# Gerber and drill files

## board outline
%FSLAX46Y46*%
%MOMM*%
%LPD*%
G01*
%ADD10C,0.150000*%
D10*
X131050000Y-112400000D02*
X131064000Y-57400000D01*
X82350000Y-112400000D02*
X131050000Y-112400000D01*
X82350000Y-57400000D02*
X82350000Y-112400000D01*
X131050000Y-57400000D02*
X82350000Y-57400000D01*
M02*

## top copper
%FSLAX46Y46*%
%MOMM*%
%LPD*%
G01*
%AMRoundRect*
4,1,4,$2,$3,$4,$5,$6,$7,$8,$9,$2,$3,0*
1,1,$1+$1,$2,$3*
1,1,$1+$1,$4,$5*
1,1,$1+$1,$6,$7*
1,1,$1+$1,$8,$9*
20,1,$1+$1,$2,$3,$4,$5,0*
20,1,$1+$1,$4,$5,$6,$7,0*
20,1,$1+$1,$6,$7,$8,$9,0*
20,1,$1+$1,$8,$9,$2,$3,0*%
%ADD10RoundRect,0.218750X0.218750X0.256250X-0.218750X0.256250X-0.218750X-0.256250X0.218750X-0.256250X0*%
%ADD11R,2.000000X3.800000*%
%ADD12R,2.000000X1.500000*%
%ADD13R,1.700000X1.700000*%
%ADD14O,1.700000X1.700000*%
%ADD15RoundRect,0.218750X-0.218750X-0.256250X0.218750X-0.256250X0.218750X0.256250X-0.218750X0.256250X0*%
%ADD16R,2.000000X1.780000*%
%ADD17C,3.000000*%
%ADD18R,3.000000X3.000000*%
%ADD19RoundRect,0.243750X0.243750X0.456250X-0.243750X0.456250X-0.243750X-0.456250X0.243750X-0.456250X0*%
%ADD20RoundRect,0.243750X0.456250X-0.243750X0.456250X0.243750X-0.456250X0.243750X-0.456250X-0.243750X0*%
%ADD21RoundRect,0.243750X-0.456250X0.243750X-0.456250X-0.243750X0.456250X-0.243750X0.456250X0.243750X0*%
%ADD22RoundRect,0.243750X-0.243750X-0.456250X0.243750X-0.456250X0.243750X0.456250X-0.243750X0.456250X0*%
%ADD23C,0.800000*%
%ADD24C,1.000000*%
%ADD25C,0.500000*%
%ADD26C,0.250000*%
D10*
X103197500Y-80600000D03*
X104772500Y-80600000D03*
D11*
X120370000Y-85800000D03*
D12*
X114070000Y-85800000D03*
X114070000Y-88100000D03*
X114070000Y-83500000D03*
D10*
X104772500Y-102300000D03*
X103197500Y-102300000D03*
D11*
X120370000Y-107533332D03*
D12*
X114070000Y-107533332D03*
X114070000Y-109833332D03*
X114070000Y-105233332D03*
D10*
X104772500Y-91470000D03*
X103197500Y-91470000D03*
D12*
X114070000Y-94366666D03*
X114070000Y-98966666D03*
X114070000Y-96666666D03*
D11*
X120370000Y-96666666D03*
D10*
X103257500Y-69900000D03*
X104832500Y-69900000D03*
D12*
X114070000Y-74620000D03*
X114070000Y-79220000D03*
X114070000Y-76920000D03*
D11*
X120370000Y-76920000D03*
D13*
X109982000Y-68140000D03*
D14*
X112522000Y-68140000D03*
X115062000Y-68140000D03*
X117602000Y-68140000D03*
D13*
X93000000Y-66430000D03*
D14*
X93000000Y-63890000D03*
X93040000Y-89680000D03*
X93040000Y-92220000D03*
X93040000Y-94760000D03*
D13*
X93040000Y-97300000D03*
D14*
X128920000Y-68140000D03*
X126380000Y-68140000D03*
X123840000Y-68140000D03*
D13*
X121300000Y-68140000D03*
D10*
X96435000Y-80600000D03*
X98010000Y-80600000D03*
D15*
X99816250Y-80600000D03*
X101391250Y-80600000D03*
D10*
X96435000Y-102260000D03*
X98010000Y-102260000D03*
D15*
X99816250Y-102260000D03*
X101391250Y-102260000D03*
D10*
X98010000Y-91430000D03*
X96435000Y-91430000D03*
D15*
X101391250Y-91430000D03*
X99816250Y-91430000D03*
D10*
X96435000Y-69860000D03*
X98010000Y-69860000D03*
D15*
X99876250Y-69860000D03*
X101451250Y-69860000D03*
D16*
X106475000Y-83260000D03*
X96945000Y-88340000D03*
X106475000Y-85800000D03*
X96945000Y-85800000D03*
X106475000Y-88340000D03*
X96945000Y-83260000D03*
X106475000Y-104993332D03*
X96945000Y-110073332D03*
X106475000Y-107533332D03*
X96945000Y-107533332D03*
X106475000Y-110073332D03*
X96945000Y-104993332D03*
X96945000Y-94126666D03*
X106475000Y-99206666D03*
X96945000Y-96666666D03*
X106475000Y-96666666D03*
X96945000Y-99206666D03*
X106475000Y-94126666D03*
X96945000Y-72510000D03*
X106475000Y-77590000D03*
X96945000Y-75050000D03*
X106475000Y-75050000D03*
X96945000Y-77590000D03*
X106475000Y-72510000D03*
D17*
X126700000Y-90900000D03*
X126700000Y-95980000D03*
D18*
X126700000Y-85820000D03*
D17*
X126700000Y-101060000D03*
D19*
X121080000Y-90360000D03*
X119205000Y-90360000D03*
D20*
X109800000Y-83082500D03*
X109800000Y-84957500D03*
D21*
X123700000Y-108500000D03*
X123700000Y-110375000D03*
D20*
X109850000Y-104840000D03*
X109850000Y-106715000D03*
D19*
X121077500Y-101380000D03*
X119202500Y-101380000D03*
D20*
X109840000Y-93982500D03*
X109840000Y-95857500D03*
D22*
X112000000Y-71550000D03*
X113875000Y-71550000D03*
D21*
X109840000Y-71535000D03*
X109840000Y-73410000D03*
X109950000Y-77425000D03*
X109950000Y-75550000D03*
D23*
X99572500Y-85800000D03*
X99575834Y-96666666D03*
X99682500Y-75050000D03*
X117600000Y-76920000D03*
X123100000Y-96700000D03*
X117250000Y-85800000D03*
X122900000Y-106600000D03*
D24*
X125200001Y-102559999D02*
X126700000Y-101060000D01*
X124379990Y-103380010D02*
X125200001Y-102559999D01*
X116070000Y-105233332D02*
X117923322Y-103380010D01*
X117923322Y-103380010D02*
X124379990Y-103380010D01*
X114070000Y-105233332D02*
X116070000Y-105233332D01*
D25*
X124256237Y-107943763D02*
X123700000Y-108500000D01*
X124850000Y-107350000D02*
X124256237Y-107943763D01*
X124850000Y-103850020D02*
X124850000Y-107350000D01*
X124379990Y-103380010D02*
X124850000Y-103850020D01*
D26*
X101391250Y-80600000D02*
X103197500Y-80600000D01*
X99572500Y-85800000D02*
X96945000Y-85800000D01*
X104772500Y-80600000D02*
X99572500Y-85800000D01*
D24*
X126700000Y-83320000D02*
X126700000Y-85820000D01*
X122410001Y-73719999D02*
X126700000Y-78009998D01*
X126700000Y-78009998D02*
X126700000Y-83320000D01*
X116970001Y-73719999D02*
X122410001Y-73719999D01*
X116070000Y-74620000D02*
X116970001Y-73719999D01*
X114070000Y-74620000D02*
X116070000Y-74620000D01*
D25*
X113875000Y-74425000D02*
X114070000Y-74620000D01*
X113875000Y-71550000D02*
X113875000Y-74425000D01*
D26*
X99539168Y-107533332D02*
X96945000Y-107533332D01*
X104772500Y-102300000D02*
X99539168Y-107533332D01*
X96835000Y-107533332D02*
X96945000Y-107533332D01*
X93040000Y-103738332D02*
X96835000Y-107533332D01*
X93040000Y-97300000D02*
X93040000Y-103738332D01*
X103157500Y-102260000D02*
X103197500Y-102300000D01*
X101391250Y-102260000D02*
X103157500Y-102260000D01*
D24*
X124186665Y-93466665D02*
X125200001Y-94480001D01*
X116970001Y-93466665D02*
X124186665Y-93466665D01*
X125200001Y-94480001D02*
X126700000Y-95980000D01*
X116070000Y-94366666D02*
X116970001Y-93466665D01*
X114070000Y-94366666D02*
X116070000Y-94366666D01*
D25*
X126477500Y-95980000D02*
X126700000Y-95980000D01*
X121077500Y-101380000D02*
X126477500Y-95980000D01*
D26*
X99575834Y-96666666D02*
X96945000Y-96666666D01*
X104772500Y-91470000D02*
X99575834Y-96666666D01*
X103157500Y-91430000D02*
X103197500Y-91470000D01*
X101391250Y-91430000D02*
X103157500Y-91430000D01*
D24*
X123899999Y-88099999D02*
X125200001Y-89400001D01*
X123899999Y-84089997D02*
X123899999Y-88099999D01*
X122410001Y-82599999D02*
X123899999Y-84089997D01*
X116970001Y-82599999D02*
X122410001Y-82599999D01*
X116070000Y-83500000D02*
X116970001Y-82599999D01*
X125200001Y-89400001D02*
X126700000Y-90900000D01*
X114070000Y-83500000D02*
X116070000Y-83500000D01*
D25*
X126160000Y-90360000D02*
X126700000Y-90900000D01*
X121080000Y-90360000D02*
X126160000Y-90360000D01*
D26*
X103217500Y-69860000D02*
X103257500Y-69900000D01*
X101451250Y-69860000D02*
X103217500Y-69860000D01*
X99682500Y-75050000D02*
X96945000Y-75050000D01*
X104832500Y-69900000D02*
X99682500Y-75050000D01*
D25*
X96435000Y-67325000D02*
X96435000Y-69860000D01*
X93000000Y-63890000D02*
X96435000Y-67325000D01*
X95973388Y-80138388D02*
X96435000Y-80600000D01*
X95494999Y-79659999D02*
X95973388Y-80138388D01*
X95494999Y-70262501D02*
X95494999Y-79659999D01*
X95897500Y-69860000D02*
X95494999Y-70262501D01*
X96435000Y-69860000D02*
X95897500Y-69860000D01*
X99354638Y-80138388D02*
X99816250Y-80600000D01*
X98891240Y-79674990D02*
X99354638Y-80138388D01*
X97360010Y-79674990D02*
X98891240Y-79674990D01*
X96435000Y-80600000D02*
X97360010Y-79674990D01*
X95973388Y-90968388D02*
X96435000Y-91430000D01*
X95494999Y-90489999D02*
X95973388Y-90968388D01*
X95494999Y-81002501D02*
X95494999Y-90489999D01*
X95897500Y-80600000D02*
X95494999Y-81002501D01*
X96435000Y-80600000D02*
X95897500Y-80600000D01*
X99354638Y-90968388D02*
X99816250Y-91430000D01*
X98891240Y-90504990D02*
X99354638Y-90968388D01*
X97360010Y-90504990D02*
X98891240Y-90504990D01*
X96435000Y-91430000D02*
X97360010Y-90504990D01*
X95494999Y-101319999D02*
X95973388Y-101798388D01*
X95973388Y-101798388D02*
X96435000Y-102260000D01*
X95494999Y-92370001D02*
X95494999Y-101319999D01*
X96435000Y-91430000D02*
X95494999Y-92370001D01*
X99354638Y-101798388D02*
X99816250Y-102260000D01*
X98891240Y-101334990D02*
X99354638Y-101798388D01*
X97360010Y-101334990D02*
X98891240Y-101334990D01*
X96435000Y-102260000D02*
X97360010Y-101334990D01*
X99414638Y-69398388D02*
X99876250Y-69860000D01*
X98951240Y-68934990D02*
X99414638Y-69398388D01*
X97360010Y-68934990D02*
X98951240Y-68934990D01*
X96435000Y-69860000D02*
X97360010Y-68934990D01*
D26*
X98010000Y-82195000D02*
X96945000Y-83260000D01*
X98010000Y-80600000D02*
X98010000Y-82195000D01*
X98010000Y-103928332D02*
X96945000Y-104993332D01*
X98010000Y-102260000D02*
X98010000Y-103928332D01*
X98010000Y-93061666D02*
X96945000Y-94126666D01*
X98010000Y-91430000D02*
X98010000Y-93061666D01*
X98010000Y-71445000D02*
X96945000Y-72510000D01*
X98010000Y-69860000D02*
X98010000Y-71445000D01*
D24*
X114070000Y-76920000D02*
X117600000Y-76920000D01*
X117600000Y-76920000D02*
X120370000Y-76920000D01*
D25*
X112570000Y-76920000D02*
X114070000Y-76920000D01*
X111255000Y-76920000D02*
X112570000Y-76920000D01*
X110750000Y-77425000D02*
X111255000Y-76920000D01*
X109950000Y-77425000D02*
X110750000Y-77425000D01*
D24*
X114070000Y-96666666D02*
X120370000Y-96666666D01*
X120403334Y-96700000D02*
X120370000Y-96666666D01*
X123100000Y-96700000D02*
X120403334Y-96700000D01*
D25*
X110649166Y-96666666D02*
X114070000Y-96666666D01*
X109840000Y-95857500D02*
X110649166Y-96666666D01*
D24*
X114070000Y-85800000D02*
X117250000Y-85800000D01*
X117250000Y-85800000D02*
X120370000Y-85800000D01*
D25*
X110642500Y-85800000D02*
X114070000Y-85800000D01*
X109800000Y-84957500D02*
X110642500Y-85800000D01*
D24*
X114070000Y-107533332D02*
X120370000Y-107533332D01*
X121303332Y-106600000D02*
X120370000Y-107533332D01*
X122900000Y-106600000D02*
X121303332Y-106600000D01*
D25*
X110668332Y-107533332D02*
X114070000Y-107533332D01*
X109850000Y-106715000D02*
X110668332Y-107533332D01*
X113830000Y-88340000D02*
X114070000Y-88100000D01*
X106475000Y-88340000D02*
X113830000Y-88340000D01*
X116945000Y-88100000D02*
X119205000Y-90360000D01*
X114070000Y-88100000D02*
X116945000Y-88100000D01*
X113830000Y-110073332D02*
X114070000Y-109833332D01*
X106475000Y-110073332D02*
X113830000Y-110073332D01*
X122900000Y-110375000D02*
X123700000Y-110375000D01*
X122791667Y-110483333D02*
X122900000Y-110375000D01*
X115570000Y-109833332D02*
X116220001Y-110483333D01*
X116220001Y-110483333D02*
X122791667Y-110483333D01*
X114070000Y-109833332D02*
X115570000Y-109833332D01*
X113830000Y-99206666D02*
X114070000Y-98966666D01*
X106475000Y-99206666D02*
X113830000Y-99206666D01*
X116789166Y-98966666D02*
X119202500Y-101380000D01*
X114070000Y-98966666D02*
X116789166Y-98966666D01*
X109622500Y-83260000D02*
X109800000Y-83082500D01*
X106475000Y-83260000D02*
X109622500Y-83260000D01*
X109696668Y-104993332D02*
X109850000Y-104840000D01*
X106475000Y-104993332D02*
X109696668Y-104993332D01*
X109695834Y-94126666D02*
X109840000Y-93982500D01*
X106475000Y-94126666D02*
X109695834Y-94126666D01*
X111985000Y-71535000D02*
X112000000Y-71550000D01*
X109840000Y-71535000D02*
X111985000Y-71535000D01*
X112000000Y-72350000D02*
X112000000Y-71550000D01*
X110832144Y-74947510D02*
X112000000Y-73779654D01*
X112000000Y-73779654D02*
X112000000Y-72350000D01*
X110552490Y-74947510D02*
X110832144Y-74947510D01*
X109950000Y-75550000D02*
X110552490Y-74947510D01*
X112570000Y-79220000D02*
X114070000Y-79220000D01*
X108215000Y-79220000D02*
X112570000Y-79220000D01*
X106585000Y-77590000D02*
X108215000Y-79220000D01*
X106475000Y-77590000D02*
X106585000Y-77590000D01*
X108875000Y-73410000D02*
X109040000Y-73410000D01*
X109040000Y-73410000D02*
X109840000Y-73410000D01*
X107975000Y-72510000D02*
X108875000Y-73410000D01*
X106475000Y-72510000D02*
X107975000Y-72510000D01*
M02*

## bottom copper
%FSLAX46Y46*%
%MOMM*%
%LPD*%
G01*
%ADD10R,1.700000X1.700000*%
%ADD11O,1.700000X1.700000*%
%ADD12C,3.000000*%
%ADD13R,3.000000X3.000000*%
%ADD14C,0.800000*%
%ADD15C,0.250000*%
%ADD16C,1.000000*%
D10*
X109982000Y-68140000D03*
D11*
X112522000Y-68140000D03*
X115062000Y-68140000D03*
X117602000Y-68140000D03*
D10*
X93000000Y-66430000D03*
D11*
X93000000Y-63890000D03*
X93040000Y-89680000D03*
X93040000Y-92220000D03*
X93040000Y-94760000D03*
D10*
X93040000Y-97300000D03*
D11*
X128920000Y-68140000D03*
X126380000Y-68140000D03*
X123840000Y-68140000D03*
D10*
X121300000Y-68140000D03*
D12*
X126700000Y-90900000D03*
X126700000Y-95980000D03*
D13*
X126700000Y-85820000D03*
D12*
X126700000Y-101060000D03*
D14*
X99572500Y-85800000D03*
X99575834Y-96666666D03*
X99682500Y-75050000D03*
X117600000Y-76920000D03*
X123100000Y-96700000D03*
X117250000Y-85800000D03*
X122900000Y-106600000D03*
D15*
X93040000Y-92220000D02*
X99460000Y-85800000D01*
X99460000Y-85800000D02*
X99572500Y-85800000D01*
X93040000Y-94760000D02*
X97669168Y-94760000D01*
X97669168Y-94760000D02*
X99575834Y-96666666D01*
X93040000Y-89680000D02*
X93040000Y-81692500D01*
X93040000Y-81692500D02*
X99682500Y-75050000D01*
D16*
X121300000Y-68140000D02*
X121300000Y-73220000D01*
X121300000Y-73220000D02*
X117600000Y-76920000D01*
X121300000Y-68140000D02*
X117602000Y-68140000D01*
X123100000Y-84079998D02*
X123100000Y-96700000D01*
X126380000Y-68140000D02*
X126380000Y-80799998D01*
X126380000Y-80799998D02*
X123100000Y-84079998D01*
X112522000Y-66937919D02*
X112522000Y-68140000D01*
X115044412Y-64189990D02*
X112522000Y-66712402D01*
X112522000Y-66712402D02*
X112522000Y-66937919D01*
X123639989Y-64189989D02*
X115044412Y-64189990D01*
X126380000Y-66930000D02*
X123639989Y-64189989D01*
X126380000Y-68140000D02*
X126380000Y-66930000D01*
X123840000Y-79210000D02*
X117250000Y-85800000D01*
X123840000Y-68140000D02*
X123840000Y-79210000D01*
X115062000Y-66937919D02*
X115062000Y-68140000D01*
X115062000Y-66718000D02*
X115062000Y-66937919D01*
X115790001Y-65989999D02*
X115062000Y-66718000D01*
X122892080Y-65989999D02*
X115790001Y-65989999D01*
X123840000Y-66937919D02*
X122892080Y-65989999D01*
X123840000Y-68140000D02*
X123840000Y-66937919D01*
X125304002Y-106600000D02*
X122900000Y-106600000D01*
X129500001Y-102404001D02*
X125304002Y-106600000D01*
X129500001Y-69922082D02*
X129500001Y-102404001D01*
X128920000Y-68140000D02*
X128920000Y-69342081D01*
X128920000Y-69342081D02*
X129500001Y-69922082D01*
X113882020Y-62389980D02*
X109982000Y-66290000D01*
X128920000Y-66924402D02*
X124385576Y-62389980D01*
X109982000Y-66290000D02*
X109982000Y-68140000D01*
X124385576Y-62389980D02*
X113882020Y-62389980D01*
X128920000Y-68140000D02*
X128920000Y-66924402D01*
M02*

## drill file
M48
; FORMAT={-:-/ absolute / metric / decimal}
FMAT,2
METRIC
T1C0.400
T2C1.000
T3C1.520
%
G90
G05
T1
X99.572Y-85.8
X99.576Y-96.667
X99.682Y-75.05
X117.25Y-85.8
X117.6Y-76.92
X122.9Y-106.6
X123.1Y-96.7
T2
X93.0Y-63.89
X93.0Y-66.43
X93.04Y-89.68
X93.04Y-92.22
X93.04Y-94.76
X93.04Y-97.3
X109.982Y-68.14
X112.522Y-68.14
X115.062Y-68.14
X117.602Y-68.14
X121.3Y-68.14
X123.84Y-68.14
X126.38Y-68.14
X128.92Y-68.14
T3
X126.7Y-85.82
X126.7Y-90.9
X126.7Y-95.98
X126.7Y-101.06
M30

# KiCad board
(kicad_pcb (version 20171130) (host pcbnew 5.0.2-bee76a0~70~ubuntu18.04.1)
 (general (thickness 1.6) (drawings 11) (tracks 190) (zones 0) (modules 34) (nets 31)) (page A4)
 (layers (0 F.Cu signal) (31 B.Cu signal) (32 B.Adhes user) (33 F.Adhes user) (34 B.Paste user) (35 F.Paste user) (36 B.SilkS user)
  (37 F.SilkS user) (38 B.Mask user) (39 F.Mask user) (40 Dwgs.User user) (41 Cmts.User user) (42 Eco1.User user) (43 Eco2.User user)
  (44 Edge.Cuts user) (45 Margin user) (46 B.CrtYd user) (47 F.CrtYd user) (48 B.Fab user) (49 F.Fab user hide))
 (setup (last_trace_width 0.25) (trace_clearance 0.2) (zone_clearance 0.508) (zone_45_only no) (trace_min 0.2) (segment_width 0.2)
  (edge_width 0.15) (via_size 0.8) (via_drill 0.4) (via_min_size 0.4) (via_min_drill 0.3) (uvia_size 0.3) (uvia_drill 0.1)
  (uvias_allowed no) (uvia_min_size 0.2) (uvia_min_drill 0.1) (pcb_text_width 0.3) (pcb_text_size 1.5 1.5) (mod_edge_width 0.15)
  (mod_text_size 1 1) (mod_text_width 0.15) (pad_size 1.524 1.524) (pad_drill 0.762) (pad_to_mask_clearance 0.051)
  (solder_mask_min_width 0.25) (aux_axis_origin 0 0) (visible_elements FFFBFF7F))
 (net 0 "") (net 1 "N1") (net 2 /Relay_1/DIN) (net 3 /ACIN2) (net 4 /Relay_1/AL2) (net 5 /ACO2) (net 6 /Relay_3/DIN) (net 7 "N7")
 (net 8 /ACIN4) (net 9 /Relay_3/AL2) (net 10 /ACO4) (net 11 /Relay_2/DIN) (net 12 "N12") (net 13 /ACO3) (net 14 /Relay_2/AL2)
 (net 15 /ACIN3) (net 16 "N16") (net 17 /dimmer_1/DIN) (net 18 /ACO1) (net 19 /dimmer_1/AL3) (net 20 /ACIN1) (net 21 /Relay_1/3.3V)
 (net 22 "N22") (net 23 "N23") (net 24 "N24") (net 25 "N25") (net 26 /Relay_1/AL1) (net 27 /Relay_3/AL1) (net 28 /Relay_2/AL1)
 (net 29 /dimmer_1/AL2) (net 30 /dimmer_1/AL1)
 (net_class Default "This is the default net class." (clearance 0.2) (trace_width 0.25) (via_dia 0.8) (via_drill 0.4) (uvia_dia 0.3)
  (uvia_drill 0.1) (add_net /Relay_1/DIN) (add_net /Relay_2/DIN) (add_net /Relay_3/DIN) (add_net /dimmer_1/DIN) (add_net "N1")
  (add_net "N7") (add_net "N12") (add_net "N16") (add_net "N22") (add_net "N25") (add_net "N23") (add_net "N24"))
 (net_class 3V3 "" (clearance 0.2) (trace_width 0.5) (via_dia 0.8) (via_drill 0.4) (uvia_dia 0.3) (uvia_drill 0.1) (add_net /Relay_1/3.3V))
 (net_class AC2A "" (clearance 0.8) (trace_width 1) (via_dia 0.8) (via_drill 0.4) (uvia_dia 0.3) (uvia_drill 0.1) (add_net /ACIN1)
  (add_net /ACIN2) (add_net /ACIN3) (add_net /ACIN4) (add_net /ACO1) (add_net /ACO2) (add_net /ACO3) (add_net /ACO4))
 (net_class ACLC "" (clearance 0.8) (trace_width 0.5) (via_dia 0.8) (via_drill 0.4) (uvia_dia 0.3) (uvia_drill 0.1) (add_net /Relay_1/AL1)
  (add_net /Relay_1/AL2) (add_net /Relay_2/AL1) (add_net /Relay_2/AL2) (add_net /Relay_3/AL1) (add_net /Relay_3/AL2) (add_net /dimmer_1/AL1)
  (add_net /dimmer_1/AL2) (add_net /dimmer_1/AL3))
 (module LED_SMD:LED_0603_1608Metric (layer F.Cu) (at 103.985 80.6 180)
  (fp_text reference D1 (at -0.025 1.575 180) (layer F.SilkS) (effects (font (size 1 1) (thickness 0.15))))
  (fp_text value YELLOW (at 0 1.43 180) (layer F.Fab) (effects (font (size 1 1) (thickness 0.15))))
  (pad 2 smd roundrect (at 0.7875 0 180) (size 0.875 0.95) (layers F.Cu F.Paste F.Mask) (roundrect_rratio 0.25) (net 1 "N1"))
  (pad 1 smd roundrect (at -0.7875 0 180) (size 0.875 0.95) (layers F.Cu F.Paste F.Mask) (roundrect_rratio 0.25) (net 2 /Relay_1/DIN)))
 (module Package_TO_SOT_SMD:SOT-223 (layer F.Cu) (at 117.22 85.8)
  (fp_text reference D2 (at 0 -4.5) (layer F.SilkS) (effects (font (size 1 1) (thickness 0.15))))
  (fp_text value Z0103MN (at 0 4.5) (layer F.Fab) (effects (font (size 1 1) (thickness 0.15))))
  (pad 4 smd rect (at 3.15 0) (size 2 3.8) (layers F.Cu F.Paste F.Mask) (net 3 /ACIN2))
  (pad 2 smd rect (at -3.15 0) (size 2 1.5) (layers F.Cu F.Paste F.Mask) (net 3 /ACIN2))
  (pad 3 smd rect (at -3.15 2.3) (size 2 1.5) (layers F.Cu F.Paste F.Mask) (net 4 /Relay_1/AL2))
  (pad 1 smd rect (at -3.15 -2.3) (size 2 1.5) (layers F.Cu F.Paste F.Mask) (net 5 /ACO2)))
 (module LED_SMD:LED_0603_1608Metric (layer F.Cu) (at 103.985 102.3 180)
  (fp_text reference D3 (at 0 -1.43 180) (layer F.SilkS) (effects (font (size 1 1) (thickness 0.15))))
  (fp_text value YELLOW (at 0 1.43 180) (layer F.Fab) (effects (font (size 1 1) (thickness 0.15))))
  (pad 1 smd roundrect (at -0.7875 0 180) (size 0.875 0.95) (layers F.Cu F.Paste F.Mask) (roundrect_rratio 0.25) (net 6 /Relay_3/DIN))
  (pad 2 smd roundrect (at 0.7875 0 180) (size 0.875 0.95) (layers F.Cu F.Paste F.Mask) (roundrect_rratio 0.25) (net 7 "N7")))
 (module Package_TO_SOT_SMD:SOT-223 (layer F.Cu) (at 117.22 107.533332)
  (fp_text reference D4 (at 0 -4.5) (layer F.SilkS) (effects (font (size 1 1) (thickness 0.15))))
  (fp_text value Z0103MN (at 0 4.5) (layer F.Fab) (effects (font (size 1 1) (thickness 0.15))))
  (pad 4 smd rect (at 3.15 0) (size 2 3.8) (layers F.Cu F.Paste F.Mask) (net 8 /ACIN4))
  (pad 2 smd rect (at -3.15 0) (size 2 1.5) (layers F.Cu F.Paste F.Mask) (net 8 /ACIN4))
  (pad 3 smd rect (at -3.15 2.3) (size 2 1.5) (layers F.Cu F.Paste F.Mask) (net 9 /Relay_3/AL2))
  (pad 1 smd rect (at -3.15 -2.3) (size 2 1.5) (layers F.Cu F.Paste F.Mask) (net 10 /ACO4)))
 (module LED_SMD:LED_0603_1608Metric (layer F.Cu) (at 103.985 91.47 180)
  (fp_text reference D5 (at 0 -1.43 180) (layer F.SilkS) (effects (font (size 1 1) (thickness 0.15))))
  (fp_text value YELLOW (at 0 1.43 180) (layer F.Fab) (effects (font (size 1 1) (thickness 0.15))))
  (pad 1 smd roundrect (at -0.7875 0 180) (size 0.875 0.95) (layers F.Cu F.Paste F.Mask) (roundrect_rratio 0.25) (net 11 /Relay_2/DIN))
  (pad 2 smd roundrect (at 0.7875 0 180) (size 0.875 0.95) (layers F.Cu F.Paste F.Mask) (roundrect_rratio 0.25) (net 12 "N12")))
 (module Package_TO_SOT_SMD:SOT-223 (layer F.Cu) (at 117.22 96.666666)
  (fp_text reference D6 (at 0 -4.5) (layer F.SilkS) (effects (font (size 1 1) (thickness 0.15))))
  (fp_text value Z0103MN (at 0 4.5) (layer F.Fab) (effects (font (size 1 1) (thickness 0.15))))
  (pad 1 smd rect (at -3.15 -2.3) (size 2 1.5) (layers F.Cu F.Paste F.Mask) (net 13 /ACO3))
  (pad 3 smd rect (at -3.15 2.3) (size 2 1.5) (layers F.Cu F.Paste F.Mask) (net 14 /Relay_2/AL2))
  (pad 2 smd rect (at -3.15 0) (size 2 1.5) (layers F.Cu F.Paste F.Mask) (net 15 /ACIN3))
  (pad 4 smd rect (at 3.15 0) (size 2 3.8) (layers F.Cu F.Paste F.Mask) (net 15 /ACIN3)))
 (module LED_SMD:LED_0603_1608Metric (layer F.Cu) (at 104.045 69.9 180)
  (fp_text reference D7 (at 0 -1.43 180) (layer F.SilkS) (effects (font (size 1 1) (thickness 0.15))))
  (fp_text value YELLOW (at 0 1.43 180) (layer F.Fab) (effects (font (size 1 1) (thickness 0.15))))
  (pad 2 smd roundrect (at 0.7875 0 180) (size 0.875 0.95) (layers F.Cu F.Paste F.Mask) (roundrect_rratio 0.25) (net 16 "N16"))
  (pad 1 smd roundrect (at -0.7875 0 180) (size 0.875 0.95) (layers F.Cu F.Paste F.Mask) (roundrect_rratio 0.25) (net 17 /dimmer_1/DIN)))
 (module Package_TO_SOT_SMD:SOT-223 (layer F.Cu) (at 117.22 76.92)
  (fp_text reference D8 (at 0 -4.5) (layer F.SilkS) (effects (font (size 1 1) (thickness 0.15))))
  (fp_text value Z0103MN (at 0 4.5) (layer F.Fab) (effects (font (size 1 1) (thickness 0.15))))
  (pad 1 smd rect (at -3.15 -2.3) (size 2 1.5) (layers F.Cu F.Paste F.Mask) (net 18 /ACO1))
  (pad 3 smd rect (at -3.15 2.3) (size 2 1.5) (layers F.Cu F.Paste F.Mask) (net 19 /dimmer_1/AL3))
  (pad 2 smd rect (at -3.15 0) (size 2 1.5) (layers F.Cu F.Paste F.Mask) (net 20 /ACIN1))
  (pad 4 smd rect (at 3.15 0) (size 2 3.8) (layers F.Cu F.Paste F.Mask) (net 20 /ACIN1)))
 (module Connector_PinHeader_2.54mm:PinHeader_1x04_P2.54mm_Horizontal (layer F.Cu) (at 109.982 68.14 90)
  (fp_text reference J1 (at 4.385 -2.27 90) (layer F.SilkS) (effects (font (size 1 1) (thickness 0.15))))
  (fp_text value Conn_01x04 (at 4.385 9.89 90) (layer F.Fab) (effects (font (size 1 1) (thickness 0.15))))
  (pad 1 thru_hole rect (at 0 0 90) (size 1.7 1.7) (drill 1) (layers *.Cu *.Mask) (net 8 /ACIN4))
  (pad 2 thru_hole oval (at 0 2.54 90) (size 1.7 1.7) (drill 1) (layers *.Cu *.Mask) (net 15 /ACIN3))
  (pad 3 thru_hole oval (at 0 5.08 90) (size 1.7 1.7) (drill 1) (layers *.Cu *.Mask) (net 3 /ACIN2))
  (pad 4 thru_hole oval (at 0 7.62 90) (size 1.7 1.7) (drill 1) (layers *.Cu *.Mask) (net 20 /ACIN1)))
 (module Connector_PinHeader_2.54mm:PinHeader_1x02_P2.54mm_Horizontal (layer F.Cu) (at 93 66.43 180)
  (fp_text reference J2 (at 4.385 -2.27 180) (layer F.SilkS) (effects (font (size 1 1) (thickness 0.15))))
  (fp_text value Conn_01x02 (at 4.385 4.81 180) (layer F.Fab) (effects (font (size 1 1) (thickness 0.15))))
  (pad 1 thru_hole rect (at 0 0 180) (size 1.7 1.7) (drill 1) (layers *.Cu *.Mask))
  (pad 2 thru_hole oval (at 0 2.54 180) (size 1.7 1.7) (drill 1) (layers *.Cu *.Mask) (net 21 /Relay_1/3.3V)))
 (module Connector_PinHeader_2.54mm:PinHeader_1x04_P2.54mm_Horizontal (layer F.Cu) (at 93.04 97.3 180)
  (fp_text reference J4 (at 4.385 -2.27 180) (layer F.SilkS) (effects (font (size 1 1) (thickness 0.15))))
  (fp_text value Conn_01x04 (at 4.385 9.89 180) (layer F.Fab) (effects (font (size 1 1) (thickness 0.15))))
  (pad 4 thru_hole oval (at 0 7.62 180) (size 1.7 1.7) (drill 1) (layers *.Cu *.Mask) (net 17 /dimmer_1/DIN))
  (pad 3 thru_hole oval (at 0 5.08 180) (size 1.7 1.7) (drill 1) (layers *.Cu *.Mask) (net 2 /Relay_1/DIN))
  (pad 2 thru_hole oval (at 0 2.54 180) (size 1.7 1.7) (drill 1) (layers *.Cu *.Mask) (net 11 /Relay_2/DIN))
  (pad 1 thru_hole rect (at 0 0 180) (size 1.7 1.7) (drill 1) (layers *.Cu *.Mask) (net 6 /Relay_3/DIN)))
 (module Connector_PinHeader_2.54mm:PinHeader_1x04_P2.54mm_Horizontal (layer F.Cu) (at 121.3 68.14 90)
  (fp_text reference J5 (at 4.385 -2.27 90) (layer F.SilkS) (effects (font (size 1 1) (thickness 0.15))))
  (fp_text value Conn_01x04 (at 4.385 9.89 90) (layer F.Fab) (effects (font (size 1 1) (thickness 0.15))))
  (pad 4 thru_hole oval (at 0 7.62 90) (size 1.7 1.7) (drill 1) (layers *.Cu *.Mask) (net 8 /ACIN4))
  (pad 3 thru_hole oval (at 0 5.08 90) (size 1.7 1.7) (drill 1) (layers *.Cu *.Mask) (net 15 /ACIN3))
  (pad 2 thru_hole oval (at 0 2.54 90) (size 1.7 1.7) (drill 1) (layers *.Cu *.Mask) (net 3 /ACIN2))
  (pad 1 thru_hole rect (at 0 0 90) (size 1.7 1.7) (drill 1) (layers *.Cu *.Mask) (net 20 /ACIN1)))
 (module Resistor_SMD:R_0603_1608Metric (layer F.Cu) (at 97.2225 80.6 180)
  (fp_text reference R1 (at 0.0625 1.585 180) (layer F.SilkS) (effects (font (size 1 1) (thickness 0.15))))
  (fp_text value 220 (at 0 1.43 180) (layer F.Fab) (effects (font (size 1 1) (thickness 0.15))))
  (pad 2 smd roundrect (at 0.7875 0 180) (size 0.875 0.95) (layers F.Cu F.Paste F.Mask) (roundrect_rratio 0.25) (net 21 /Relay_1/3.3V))
  (pad 1 smd roundrect (at -0.7875 0 180) (size 0.875 0.95) (layers F.Cu F.Paste F.Mask) (roundrect_rratio 0.25) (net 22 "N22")))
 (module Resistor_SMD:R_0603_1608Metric (layer F.Cu) (at 100.60375 80.6)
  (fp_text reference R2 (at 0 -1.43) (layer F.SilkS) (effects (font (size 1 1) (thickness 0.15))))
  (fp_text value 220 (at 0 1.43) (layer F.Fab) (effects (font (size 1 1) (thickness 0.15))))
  (pad 1 smd roundrect (at -0.7875 0) (size 0.875 0.95) (layers F.Cu F.Paste F.Mask) (roundrect_rratio 0.25) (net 21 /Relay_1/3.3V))
  (pad 2 smd roundrect (at 0.7875 0) (size 0.875 0.95) (layers F.Cu F.Paste F.Mask) (roundrect_rratio 0.25) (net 1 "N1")))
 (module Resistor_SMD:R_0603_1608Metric (layer F.Cu) (at 97.2225 102.26 180)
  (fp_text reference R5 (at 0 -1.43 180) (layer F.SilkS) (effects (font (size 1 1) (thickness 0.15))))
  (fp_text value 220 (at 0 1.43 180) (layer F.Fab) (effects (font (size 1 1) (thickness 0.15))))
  (pad 2 smd roundrect (at 0.7875 0 180) (size 0.875 0.95) (layers F.Cu F.Paste F.Mask) (roundrect_rratio 0.25) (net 21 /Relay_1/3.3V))
  (pad 1 smd roundrect (at -0.7875 0 180) (size 0.875 0.95) (layers F.Cu F.Paste F.Mask) (roundrect_rratio 0.25) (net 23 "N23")))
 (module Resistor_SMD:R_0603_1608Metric (layer F.Cu) (at 100.60375 102.26)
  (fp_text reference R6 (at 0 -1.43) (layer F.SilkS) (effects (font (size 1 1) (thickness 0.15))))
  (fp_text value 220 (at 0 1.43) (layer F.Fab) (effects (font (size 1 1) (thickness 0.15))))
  (pad 1 smd roundrect (at -0.7875 0) (size 0.875 0.95) (layers F.Cu F.Paste F.Mask) (roundrect_rratio 0.25) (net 21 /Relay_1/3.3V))
  (pad 2 smd roundrect (at 0.7875 0) (size 0.875 0.95) (layers F.Cu F.Paste F.Mask) (roundrect_rratio 0.25) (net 7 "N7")))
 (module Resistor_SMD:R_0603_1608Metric (layer F.Cu) (at 97.2225 91.43 180)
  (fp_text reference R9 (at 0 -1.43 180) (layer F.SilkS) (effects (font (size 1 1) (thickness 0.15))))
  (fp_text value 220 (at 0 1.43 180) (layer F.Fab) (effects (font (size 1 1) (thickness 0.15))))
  (pad 1 smd roundrect (at -0.7875 0 180) (size 0.875 0.95) (layers F.Cu F.Paste F.Mask) (roundrect_rratio 0.25) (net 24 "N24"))
  (pad 2 smd roundrect (at 0.7875 0 180) (size 0.875 0.95) (layers F.Cu F.Paste F.Mask) (roundrect_rratio 0.25) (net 21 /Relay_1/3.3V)))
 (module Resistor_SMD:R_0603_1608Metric (layer F.Cu) (at 100.60375 91.43)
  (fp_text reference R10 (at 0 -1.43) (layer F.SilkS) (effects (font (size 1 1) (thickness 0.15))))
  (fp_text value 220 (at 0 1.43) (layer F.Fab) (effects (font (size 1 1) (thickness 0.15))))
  (pad 2 smd roundrect (at 0.7875 0) (size 0.875 0.95) (layers F.Cu F.Paste F.Mask) (roundrect_rratio 0.25) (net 12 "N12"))
  (pad 1 smd roundrect (at -0.7875 0) (size 0.875 0.95) (layers F.Cu F.Paste F.Mask) (roundrect_rratio 0.25) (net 21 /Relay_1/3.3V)))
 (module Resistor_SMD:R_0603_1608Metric (layer F.Cu) (at 97.2225 69.86 180)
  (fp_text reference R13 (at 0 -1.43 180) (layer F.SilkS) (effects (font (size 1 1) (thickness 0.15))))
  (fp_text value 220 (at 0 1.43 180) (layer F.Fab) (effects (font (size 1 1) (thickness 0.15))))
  (pad 2 smd roundrect (at 0.7875 0 180) (size 0.875 0.95) (layers F.Cu F.Paste F.Mask) (roundrect_rratio 0.25) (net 21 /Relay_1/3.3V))
  (pad 1 smd roundrect (at -0.7875 0 180) (size 0.875 0.95) (layers F.Cu F.Paste F.Mask) (roundrect_rratio 0.25) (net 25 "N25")))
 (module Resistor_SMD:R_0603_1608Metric (layer F.Cu) (at 100.66375 69.86)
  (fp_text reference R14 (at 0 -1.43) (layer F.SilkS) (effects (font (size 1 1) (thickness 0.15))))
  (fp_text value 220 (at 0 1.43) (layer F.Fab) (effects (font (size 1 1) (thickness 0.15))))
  (pad 1 smd roundrect (at -0.7875 0) (size 0.875 0.95) (layers F.Cu F.Paste F.Mask) (roundrect_rratio 0.25) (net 21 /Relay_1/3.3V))
  (pad 2 smd roundrect (at 0.7875 0) (size 0.875 0.95) (layers F.Cu F.Paste F.Mask) (roundrect_rratio 0.25) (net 16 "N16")))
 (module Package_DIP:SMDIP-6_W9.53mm (layer F.Cu) (at 101.71 85.8)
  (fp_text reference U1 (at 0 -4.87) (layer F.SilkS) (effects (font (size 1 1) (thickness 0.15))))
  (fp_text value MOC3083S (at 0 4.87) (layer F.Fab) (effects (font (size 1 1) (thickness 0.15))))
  (pad 6 smd rect (at 4.765 -2.54) (size 2 1.78) (layers F.Cu F.Paste F.Mask) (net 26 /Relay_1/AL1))
  (pad 3 smd rect (at -4.765 2.54) (size 2 1.78) (layers F.Cu F.Paste F.Mask))
  (pad 5 smd rect (at 4.765 0) (size 2 1.78) (layers F.Cu F.Paste F.Mask))
  (pad 2 smd rect (at -4.765 0) (size 2 1.78) (layers F.Cu F.Paste F.Mask) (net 2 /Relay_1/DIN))
  (pad 4 smd rect (at 4.765 2.54) (size 2 1.78) (layers F.Cu F.Paste F.Mask) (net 4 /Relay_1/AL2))
  (pad 1 smd rect (at -4.765 -2.54) (size 2 1.78) (layers F.Cu F.Paste F.Mask) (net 22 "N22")))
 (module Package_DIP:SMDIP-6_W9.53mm (layer F.Cu) (at 101.71 107.533332)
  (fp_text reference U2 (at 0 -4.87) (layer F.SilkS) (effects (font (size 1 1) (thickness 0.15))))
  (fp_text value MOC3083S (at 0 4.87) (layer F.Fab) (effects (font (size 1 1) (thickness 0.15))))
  (pad 6 smd rect (at 4.765 -2.54) (size 2 1.78) (layers F.Cu F.Paste F.Mask) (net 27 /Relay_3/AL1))
  (pad 3 smd rect (at -4.765 2.54) (size 2 1.78) (layers F.Cu F.Paste F.Mask))
  (pad 5 smd rect (at 4.765 0) (size 2 1.78) (layers F.Cu F.Paste F.Mask))
  (pad 2 smd rect (at -4.765 0) (size 2 1.78) (layers F.Cu F.Paste F.Mask) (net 6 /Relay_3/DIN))
  (pad 4 smd rect (at 4.765 2.54) (size 2 1.78) (layers F.Cu F.Paste F.Mask) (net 9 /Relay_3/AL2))
  (pad 1 smd rect (at -4.765 -2.54) (size 2 1.78) (layers F.Cu F.Paste F.Mask) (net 23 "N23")))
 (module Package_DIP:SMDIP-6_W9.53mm (layer F.Cu) (at 101.71 96.666666)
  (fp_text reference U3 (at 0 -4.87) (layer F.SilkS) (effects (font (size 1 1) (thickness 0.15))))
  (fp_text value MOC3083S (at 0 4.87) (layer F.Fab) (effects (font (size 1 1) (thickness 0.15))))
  (pad 1 smd rect (at -4.765 -2.54) (size 2 1.78) (layers F.Cu F.Paste F.Mask) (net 24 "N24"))
  (pad 4 smd rect (at 4.765 2.54) (size 2 1.78) (layers F.Cu F.Paste F.Mask) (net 14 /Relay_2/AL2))
  (pad 2 smd rect (at -4.765 0) (size 2 1.78) (layers F.Cu F.Paste F.Mask) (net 11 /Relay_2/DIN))
  (pad 5 smd rect (at 4.765 0) (size 2 1.78) (layers F.Cu F.Paste F.Mask))
  (pad 3 smd rect (at -4.765 2.54) (size 2 1.78) (layers F.Cu F.Paste F.Mask))
  (pad 6 smd rect (at 4.765 -2.54) (size 2 1.78) (layers F.Cu F.Paste F.Mask) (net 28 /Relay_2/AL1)))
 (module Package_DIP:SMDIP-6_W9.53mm (layer F.Cu) (at 101.71 75.05)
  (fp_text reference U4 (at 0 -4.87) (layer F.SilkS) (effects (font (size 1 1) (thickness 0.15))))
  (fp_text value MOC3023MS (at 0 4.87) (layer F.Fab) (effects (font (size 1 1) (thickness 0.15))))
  (pad 1 smd rect (at -4.765 -2.54) (size 2 1.78) (layers F.Cu F.Paste F.Mask) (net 25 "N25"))
  (pad 4 smd rect (at 4.765 2.54) (size 2 1.78) (layers F.Cu F.Paste F.Mask) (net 19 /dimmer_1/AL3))
  (pad 2 smd rect (at -4.765 0) (size 2 1.78) (layers F.Cu F.Paste F.Mask) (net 17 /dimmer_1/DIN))
  (pad 5 smd rect (at 4.765 0) (size 2 1.78) (layers F.Cu F.Paste F.Mask))
  (pad 3 smd rect (at -4.765 2.54) (size 2 1.78) (layers F.Cu F.Paste F.Mask))
  (pad 6 smd rect (at 4.765 -2.54) (size 2 1.78) (layers F.Cu F.Paste F.Mask) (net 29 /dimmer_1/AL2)))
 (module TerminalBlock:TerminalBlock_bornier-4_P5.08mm (layer F.Cu) (at 126.7 85.82 270)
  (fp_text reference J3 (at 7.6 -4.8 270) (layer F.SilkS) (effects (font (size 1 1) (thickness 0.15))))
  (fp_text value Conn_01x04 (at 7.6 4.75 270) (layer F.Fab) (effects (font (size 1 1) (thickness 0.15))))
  (pad 2 thru_hole circle (at 5.08 0 270) (size 3 3) (drill 1.52) (layers *.Cu *.Mask) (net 5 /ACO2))
  (pad 3 thru_hole circle (at 10.16 0 270) (size 3 3) (drill 1.52) (layers *.Cu *.Mask) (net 13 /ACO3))
  (pad 1 thru_hole rect (at 0 0 270) (size 3 3) (drill 1.52) (layers *.Cu *.Mask) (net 18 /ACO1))
  (pad 4 thru_hole circle (at 15.24 0 270) (size 3 3) (drill 1.52) (layers *.Cu *.Mask) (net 10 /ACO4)))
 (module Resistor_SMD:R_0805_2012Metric (layer F.Cu) (at 120.1425 90.36 180)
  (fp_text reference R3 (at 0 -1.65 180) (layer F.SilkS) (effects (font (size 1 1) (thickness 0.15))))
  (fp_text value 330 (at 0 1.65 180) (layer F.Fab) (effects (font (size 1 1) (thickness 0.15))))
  (pad 1 smd roundrect (at -0.9375 0 180) (size 0.975 1.4) (layers F.Cu F.Paste F.Mask) (roundrect_rratio 0.25) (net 5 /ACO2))
  (pad 2 smd roundrect (at 0.9375 0 180) (size 0.975 1.4) (layers F.Cu F.Paste F.Mask) (roundrect_rratio 0.25) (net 4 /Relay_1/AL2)))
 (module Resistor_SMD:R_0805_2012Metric (layer F.Cu) (at 109.8 84.02 90)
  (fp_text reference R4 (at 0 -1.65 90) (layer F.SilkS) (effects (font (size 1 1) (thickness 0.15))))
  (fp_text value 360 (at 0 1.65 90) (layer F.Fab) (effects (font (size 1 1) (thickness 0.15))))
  (pad 2 smd roundrect (at 0.9375 0 90) (size 0.975 1.4) (layers F.Cu F.Paste F.Mask) (roundrect_rratio 0.25) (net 26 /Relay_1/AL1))
  (pad 1 smd roundrect (at -0.9375 0 90) (size 0.975 1.4) (layers F.Cu F.Paste F.Mask) (roundrect_rratio 0.25) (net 3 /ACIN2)))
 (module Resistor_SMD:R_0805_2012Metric (layer F.Cu) (at 123.7 109.4375 270)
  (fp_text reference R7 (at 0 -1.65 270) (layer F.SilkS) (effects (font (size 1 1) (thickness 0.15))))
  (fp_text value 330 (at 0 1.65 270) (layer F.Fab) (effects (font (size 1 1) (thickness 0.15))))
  (pad 1 smd roundrect (at -0.9375 0 270) (size 0.975 1.4) (layers F.Cu F.Paste F.Mask) (roundrect_rratio 0.25) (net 10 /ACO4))
  (pad 2 smd roundrect (at 0.9375 0 270) (size 0.975 1.4) (layers F.Cu F.Paste F.Mask) (roundrect_rratio 0.25) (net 9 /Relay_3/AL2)))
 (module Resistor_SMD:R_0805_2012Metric (layer F.Cu) (at 109.85 105.7775 90)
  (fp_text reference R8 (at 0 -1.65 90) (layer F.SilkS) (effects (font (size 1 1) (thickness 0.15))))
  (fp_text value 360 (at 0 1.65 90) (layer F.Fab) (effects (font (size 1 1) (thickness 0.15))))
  (pad 2 smd roundrect (at 0.9375 0 90) (size 0.975 1.4) (layers F.Cu F.Paste F.Mask) (roundrect_rratio 0.25) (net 27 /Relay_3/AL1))
  (pad 1 smd roundrect (at -0.9375 0 90) (size 0.975 1.4) (layers F.Cu F.Paste F.Mask) (roundrect_rratio 0.25) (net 8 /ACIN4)))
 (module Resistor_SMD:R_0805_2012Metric (layer F.Cu) (at 120.14 101.38 180)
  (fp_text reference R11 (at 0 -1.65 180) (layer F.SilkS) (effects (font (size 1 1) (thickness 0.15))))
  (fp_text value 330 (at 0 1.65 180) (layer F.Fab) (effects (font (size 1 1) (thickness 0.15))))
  (pad 1 smd roundrect (at -0.9375 0 180) (size 0.975 1.4) (layers F.Cu F.Paste F.Mask) (roundrect_rratio 0.25) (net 13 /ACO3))
  (pad 2 smd roundrect (at 0.9375 0 180) (size 0.975 1.4) (layers F.Cu F.Paste F.Mask) (roundrect_rratio 0.25) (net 14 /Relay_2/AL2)))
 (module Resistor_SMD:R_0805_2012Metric (layer F.Cu) (at 109.84 94.92 90)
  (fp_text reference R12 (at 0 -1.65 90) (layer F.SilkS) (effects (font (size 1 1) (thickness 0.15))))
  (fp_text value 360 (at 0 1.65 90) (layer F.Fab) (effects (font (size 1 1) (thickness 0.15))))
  (pad 2 smd roundrect (at 0.9375 0 90) (size 0.975 1.4) (layers F.Cu F.Paste F.Mask) (roundrect_rratio 0.25) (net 28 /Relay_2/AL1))
  (pad 1 smd roundrect (at -0.9375 0 90) (size 0.975 1.4) (layers F.Cu F.Paste F.Mask) (roundrect_rratio 0.25) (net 15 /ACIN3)))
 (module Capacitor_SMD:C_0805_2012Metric (layer F.Cu) (at 112.9375 71.55)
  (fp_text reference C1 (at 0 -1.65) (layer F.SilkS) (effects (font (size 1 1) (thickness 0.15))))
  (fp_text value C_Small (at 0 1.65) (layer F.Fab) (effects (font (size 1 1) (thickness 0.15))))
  (pad 1 smd roundrect (at -0.9375 0) (size 0.975 1.4) (layers F.Cu F.Paste F.Mask) (roundrect_rratio 0.25) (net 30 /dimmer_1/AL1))
  (pad 2 smd roundrect (at 0.9375 0) (size 0.975 1.4) (layers F.Cu F.Paste F.Mask) (roundrect_rratio 0.25) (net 18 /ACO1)))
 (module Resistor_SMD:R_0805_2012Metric (layer F.Cu) (at 109.84 72.4725 270)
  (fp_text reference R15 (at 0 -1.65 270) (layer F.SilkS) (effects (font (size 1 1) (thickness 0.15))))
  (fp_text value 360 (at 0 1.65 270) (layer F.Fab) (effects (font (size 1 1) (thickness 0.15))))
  (pad 1 smd roundrect (at -0.9375 0 270) (size 0.975 1.4) (layers F.Cu F.Paste F.Mask) (roundrect_rratio 0.25) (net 30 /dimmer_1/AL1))
  (pad 2 smd roundrect (at 0.9375 0 270) (size 0.975 1.4) (layers F.Cu F.Paste F.Mask) (roundrect_rratio 0.25) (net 29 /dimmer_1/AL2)))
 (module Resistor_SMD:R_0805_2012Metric (layer F.Cu) (at 109.95 76.4875 270)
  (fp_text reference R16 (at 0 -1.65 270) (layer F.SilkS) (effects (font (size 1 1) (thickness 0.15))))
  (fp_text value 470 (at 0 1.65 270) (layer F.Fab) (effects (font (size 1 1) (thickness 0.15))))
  (pad 2 smd roundrect (at 0.9375 0 270) (size 0.975 1.4) (layers F.Cu F.Paste F.Mask) (roundrect_rratio 0.25) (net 20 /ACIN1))
  (pad 1 smd roundrect (at -0.9375 0 270) (size 0.975 1.4) (layers F.Cu F.Paste F.Mask) (roundrect_rratio 0.25) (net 30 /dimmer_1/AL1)))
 (gr_line (start 131.05 112.4) (end 131.064 57.4) (layer Edge.Cuts) (width 0.15))
 (gr_line (start 82.35 112.4) (end 131.05 112.4) (layer Edge.Cuts) (width 0.15))
 (gr_line (start 82.35 57.4) (end 82.35 112.4) (layer Edge.Cuts) (width 0.15))
 (gr_line (start 131.05 57.4) (end 82.35 57.4) (layer Edge.Cuts) (width 0.15))
 (segment (start 125.200001 102.559999) (end 126.7 101.06) (width 1) (layer F.Cu) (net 10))
 (segment (start 124.37999 103.38001) (end 125.200001 102.559999) (width 1) (layer F.Cu) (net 10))
 (segment (start 116.07 105.233332) (end 117.923322 103.38001) (width 1) (layer F.Cu) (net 10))
 (segment (start 117.923322 103.38001) (end 124.37999 103.38001) (width 1) (layer F.Cu) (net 10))
 (segment (start 114.07 105.233332) (end 116.07 105.233332) (width 1) (layer F.Cu) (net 10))
 (segment (start 124.256237 107.943763) (end 123.7 108.5) (width 0.5) (layer F.Cu) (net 10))
 (segment (start 124.85 107.35) (end 124.256237 107.943763) (width 0.5) (layer F.Cu) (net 10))
 (segment (start 124.85 103.85002) (end 124.85 107.35) (width 0.5) (layer F.Cu) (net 10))
 (segment (start 124.37999 103.38001) (end 124.85 103.85002) (width 0.5) (layer F.Cu) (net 10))
 (segment (start 101.39125 80.6) (end 103.1975 80.6) (width 0.25) (layer F.Cu) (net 1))
 (segment (start 99.5725 85.8) (end 96.945 85.8) (width 0.25) (layer F.Cu) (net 2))
 (segment (start 104.7725 80.6) (end 99.5725 85.8) (width 0.25) (layer F.Cu) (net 2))
 (via (at 99.5725 85.8) (size 0.8) (drill 0.4) (layers F.Cu B.Cu) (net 2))
 (segment (start 93.04 92.22) (end 99.46 85.8) (width 0.25) (layer B.Cu) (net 2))
 (segment (start 99.46 85.8) (end 99.5725 85.8) (width 0.25) (layer B.Cu) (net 2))
 (segment (start 126.7 83.32) (end 126.7 85.82) (width 1) (layer F.Cu) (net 18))
 (segment (start 122.410001 73.719999) (end 126.7 78.009998) (width 1) (layer F.Cu) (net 18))
 (segment (start 126.7 78.009998) (end 126.7 83.32) (width 1) (layer F.Cu) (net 18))
 (segment (start 116.970001 73.719999) (end 122.410001 73.719999) (width 1) (layer F.Cu) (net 18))
 (segment (start 116.07 74.62) (end 116.970001 73.719999) (width 1) (layer F.Cu) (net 18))
 (segment (start 114.07 74.62) (end 116.07 74.62) (width 1) (layer F.Cu) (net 18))
 (segment (start 113.875 74.425) (end 114.07 74.62) (width 0.5) (layer F.Cu) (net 18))
 (segment (start 113.875 71.55) (end 113.875 74.425) (width 0.5) (layer F.Cu) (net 18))
 (segment (start 99.539168 107.533332) (end 96.945 107.533332) (width 0.25) (layer F.Cu) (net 6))
 (segment (start 104.7725 102.3) (end 99.539168 107.533332) (width 0.25) (layer F.Cu) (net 6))
 (segment (start 96.835 107.533332) (end 96.945 107.533332) (width 0.25) (layer F.Cu) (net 6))
 (segment (start 93.04 103.738332) (end 96.835 107.533332) (width 0.25) (layer F.Cu) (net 6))
 (segment (start 93.04 97.3) (end 93.04 103.738332) (width 0.25) (layer F.Cu) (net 6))
 (segment (start 103.1575 102.26) (end 103.1975 102.3) (width 0.25) (layer F.Cu) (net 7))
 (segment (start 101.39125 102.26) (end 103.1575 102.26) (width 0.25) (layer F.Cu) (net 7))
 (segment (start 124.186665 93.466665) (end 125.200001 94.480001) (width 1) (layer F.Cu) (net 13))
 (segment (start 116.970001 93.466665) (end 124.186665 93.466665) (width 1) (layer F.Cu) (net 13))
 (segment (start 125.200001 94.480001) (end 126.7 95.98) (width 1) (layer F.Cu) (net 13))
 (segment (start 116.07 94.366666) (end 116.970001 93.466665) (width 1) (layer F.Cu) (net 13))
 (segment (start 114.07 94.366666) (end 116.07 94.366666) (width 1) (layer F.Cu) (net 13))
 (segment (start 126.4775 95.98) (end 126.7 95.98) (width 0.5) (layer F.Cu) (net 13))
 (segment (start 121.0775 101.38) (end 126.4775 95.98) (width 0.5) (layer F.Cu) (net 13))
 (segment (start 99.575834 96.666666) (end 96.945 96.666666) (width 0.25) (layer F.Cu) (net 11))
 (segment (start 104.7725 91.47) (end 99.575834 96.666666) (width 0.25) (layer F.Cu) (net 11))
 (via (at 99.575834 96.666666) (size 0.8) (drill 0.4) (layers F.Cu B.Cu) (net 11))
 (segment (start 93.04 94.76) (end 97.669168 94.76) (width 0.25) (layer B.Cu) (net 11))
 (segment (start 97.669168 94.76) (end 99.575834 96.666666) (width 0.25) (layer B.Cu) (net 11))
 (segment (start 103.1575 91.43) (end 103.1975 91.47) (width 0.25) (layer F.Cu) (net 12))
 (segment (start 101.39125 91.43) (end 103.1575 91.43) (width 0.25) (layer F.Cu) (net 12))
 (segment (start 123.899999 88.099999) (end 125.200001 89.400001) (width 1) (layer F.Cu) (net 5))
 (segment (start 123.899999 84.089997) (end 123.899999 88.099999) (width 1) (layer F.Cu) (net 5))
 (segment (start 122.410001 82.599999) (end 123.899999 84.089997) (width 1) (layer F.Cu) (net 5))
 (segment (start 116.970001 82.599999) (end 122.410001 82.599999) (width 1) (layer F.Cu) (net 5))
 (segment (start 116.07 83.5) (end 116.970001 82.599999) (width 1) (layer F.Cu) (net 5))
 (segment (start 125.200001 89.400001) (end 126.7 90.9) (width 1) (layer F.Cu) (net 5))
 (segment (start 114.07 83.5) (end 116.07 83.5) (width 1) (layer F.Cu) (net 5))
 (segment (start 126.16 90.36) (end 126.7 90.9) (width 0.5) (layer F.Cu) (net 5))
 (segment (start 121.08 90.36) (end 126.16 90.36) (width 0.5) (layer F.Cu) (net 5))
 (segment (start 103.2175 69.86) (end 103.2575 69.9) (width 0.25) (layer F.Cu) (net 16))
 (segment (start 101.45125 69.86) (end 103.2175 69.86) (width 0.25) (layer F.Cu) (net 16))
 (segment (start 99.6825 75.05) (end 96.945 75.05) (width 0.25) (layer F.Cu) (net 17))
 (segment (start 104.8325 69.9) (end 99.6825 75.05) (width 0.25) (layer F.Cu) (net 17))
 (via (at 99.6825 75.05) (size 0.8) (drill 0.4) (layers F.Cu B.Cu) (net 17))
 (segment (start 93.04 89.68) (end 93.04 81.6925) (width 0.25) (layer B.Cu) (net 17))
 (segment (start 93.04 81.6925) (end 99.6825 75.05) (width 0.25) (layer B.Cu) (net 17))
 (segment (start 96.435 67.325) (end 96.435 69.86) (width 0.5) (layer F.Cu) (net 21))
 (segment (start 93 63.89) (end 96.435 67.325) (width 0.5) (layer F.Cu) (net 21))
 (segment (start 95.973388 80.138388) (end 96.435 80.6) (width 0.5) (layer F.Cu) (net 21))
 (segment (start 95.494999 79.659999) (end 95.973388 80.138388) (width 0.5) (layer F.Cu) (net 21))
 (segment (start 95.494999 70.262501) (end 95.494999 79.659999) (width 0.5) (layer F.Cu) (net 21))
 (segment (start 95.8975 69.86) (end 95.494999 70.262501) (width 0.5) (layer F.Cu) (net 21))
 (segment (start 96.435 69.86) (end 95.8975 69.86) (width 0.5) (layer F.Cu) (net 21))
 (segment (start 99.354638 80.138388) (end 99.81625 80.6) (width 0.5) (layer F.Cu) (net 21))
 (segment (start 98.89124 79.67499) (end 99.354638 80.138388) (width 0.5) (layer F.Cu) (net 21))
 (segment (start 97.36001 79.67499) (end 98.89124 79.67499) (width 0.5) (layer F.Cu) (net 21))
 (segment (start 96.435 80.6) (end 97.36001 79.67499) (width 0.5) (layer F.Cu) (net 21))
 (segment (start 95.973388 90.968388) (end 96.435 91.43) (width 0.5) (layer F.Cu) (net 21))
 (segment (start 95.494999 90.489999) (end 95.973388 90.968388) (width 0.5) (layer F.Cu) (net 21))
 (segment (start 95.494999 81.002501) (end 95.494999 90.489999) (width 0.5) (layer F.Cu) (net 21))
 (segment (start 95.8975 80.6) (end 95.494999 81.002501) (width 0.5) (layer F.Cu) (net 21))
 (segment (start 96.435 80.6) (end 95.8975 80.6) (width 0.5) (layer F.Cu) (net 21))
 (segment (start 99.354638 90.968388) (end 99.81625 91.43) (width 0.5) (layer F.Cu) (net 21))
 (segment (start 98.89124 90.50499) (end 99.354638 90.968388) (width 0.5) (layer F.Cu) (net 21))
 (segment (start 97.36001 90.50499) (end 98.89124 90.50499) (width 0.5) (layer F.Cu) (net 21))
 (segment (start 96.435 91.43) (end 97.36001 90.50499) (width 0.5) (layer F.Cu) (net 21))
 (segment (start 95.494999 101.319999) (end 95.973388 101.798388) (width 0.5) (layer F.Cu) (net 21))
 (segment (start 95.973388 101.798388) (end 96.435 102.26) (width 0.5) (layer F.Cu) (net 21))
 (segment (start 95.494999 92.370001) (end 95.494999 101.319999) (width 0.5) (layer F.Cu) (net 21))
 (segment (start 96.435 91.43) (end 95.494999 92.370001) (width 0.5) (layer F.Cu) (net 21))
 (segment (start 99.354638 101.798388) (end 99.81625 102.26) (width 0.5) (layer F.Cu) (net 21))
 (segment (start 98.89124 101.33499) (end 99.354638 101.798388) (width 0.5) (layer F.Cu) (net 21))
 (segment (start 97.36001 101.33499) (end 98.89124 101.33499) (width 0.5) (layer F.Cu) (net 21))
 (segment (start 96.435 102.26) (end 97.36001 101.33499) (width 0.5) (layer F.Cu) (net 21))
 (segment (start 99.414638 69.398388) (end 99.87625 69.86) (width 0.5) (layer F.Cu) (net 21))
 (segment (start 98.95124 68.93499) (end 99.414638 69.398388) (width 0.5) (layer F.Cu) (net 21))
 (segment (start 97.36001 68.93499) (end 98.95124 68.93499) (width 0.5) (layer F.Cu) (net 21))
 (segment (start 96.435 69.86) (end 97.36001 68.93499) (width 0.5) (layer F.Cu) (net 21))
 (segment (start 98.01 82.195) (end 96.945 83.26) (width 0.25) (layer F.Cu) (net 22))
 (segment (start 98.01 80.6) (end 98.01 82.195) (width 0.25) (layer F.Cu) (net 22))
 (segment (start 98.01 103.928332) (end 96.945 104.993332) (width 0.25) (layer F.Cu) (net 23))
 (segment (start 98.01 102.26) (end 98.01 103.928332) (width 0.25) (layer F.Cu) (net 23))
 (segment (start 98.01 93.061666) (end 96.945 94.126666) (width 0.25) (layer F.Cu) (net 24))
 (segment (start 98.01 91.43) (end 98.01 93.061666) (width 0.25) (layer F.Cu) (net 24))
 (segment (start 98.01 71.445) (end 96.945 72.51) (width 0.25) (layer F.Cu) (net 25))
 (segment (start 98.01 69.86) (end 98.01 71.445) (width 0.25) (layer F.Cu) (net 25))
 (segment (start 114.07 76.92) (end 117.6 76.92) (width 1) (layer F.Cu) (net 20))
 (segment (start 117.6 76.92) (end 120.37 76.92) (width 1) (layer F.Cu) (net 20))
 (via (at 117.6 76.92) (size 0.8) (drill 0.4) (layers F.Cu B.Cu) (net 20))
 (segment (start 121.3 68.14) (end 121.3 73.22) (width 1) (layer B.Cu) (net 20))
 (segment (start 121.3 73.22) (end 117.6 76.92) (width 1) (layer B.Cu) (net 20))
 (segment (start 112.57 76.92) (end 114.07 76.92) (width 0.5) (layer F.Cu) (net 20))
 (segment (start 111.255 76.92) (end 112.57 76.92) (width 0.5) (layer F.Cu) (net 20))
 (segment (start 110.75 77.425) (end 111.255 76.92) (width 0.5) (layer F.Cu) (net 20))
 (segment (start 109.95 77.425) (end 110.75 77.425) (width 0.5) (layer F.Cu) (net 20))
 (segment (start 121.3 68.14) (end 117.602 68.14) (width 1) (layer B.Cu) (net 20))
 (segment (start 114.07 96.666666) (end 120.37 96.666666) (width 1) (layer F.Cu) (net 15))
 (segment (start 123.1 84.079998) (end 123.1 96.7) (width 1) (layer B.Cu) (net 15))
 (segment (start 126.38 68.14) (end 126.38 80.799998) (width 1) (layer B.Cu) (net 15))
 (via (at 123.1 96.7) (size 0.8) (drill 0.4) (layers F.Cu B.Cu) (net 15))
 (segment (start 126.38 80.799998) (end 123.1 84.079998) (width 1) (layer B.Cu) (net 15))
 (segment (start 120.403334 96.7) (end 120.37 96.666666) (width 1) (layer F.Cu) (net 15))
 (segment (start 123.1 96.7) (end 120.403334 96.7) (width 1) (layer F.Cu) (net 15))
 (segment (start 110.649166 96.666666) (end 114.07 96.666666) (width 0.5) (layer F.Cu) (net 15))
 (segment (start 109.84 95.8575) (end 110.649166 96.666666) (width 0.5) (layer F.Cu) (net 15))
 (segment (start 112.522 66.937919) (end 112.522 68.14) (width 1) (layer B.Cu) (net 15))
 (segment (start 115.044412 64.18999) (end 112.522 66.712402) (width 1) (layer B.Cu) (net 15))
 (segment (start 112.522 66.712402) (end 112.522 66.937919) (width 1) (layer B.Cu) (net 15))
 (segment (start 123.639989 64.189989) (end 115.044412 64.18999) (width 1) (layer B.Cu) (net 15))
 (segment (start 126.38 66.93) (end 123.639989 64.189989) (width 1) (layer B.Cu) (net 15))
 (segment (start 126.38 68.14) (end 126.38 66.93) (width 1) (layer B.Cu) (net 15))
 (via (at 117.25 85.8) (size 0.8) (drill 0.4) (layers F.Cu B.Cu) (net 3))
 (segment (start 123.84 79.21) (end 117.25 85.8) (width 1) (layer B.Cu) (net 3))
 (segment (start 123.84 68.14) (end 123.84 79.21) (width 1) (layer B.Cu) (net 3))
 (segment (start 114.07 85.8) (end 117.25 85.8) (width 1) (layer F.Cu) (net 3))
 (segment (start 117.25 85.8) (end 120.37 85.8) (width 1) (layer F.Cu) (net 3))
 (segment (start 110.6425 85.8) (end 114.07 85.8) (width 0.5) (layer F.Cu) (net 3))
 (segment (start 109.8 84.9575) (end 110.6425 85.8) (width 0.5) (layer F.Cu) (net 3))
 (segment (start 115.062 66.937919) (end 115.062 68.14) (width 1) (layer B.Cu) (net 3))
 (segment (start 115.062 66.718) (end 115.062 66.937919) (width 1) (layer B.Cu) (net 3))
 (segment (start 115.790001 65.989999) (end 115.062 66.718) (width 1) (layer B.Cu) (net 3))
 (segment (start 122.89208 65.989999) (end 115.790001 65.989999) (width 1) (layer B.Cu) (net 3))
 (segment (start 123.84 66.937919) (end 122.89208 65.989999) (width 1) (layer B.Cu) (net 3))
 (segment (start 123.84 68.14) (end 123.84 66.937919) (width 1) (layer B.Cu) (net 3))
 (segment (start 114.07 107.533332) (end 120.37 107.533332) (width 1) (layer F.Cu) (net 8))
 (via (at 122.9 106.6) (size 0.8) (drill 0.4) (layers F.Cu B.Cu) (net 8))
 (segment (start 125.304002 106.6) (end 122.9 106.6) (width 1) (layer B.Cu) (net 8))
 (segment (start 129.500001 102.404001) (end 125.304002 106.6) (width 1) (layer B.Cu) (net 8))
 (segment (start 129.500001 69.922082) (end 129.500001 102.404001) (width 1) (layer B.Cu) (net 8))
 (segment (start 128.92 68.14) (end 128.92 69.342081) (width 1) (layer B.Cu) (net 8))
 (segment (start 128.92 69.342081) (end 129.500001 69.922082) (width 1) (layer B.Cu) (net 8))
 (segment (start 121.303332 106.6) (end 120.37 107.533332) (width 1) (layer F.Cu) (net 8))
 (segment (start 122.9 106.6) (end 121.303332 106.6) (width 1) (layer F.Cu) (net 8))
 (segment (start 110.668332 107.533332) (end 114.07 107.533332) (width 0.5) (layer F.Cu) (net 8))
 (segment (start 109.85 106.715) (end 110.668332 107.533332) (width 0.5) (layer F.Cu) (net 8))
 (segment (start 113.88202 62.38998) (end 109.982 66.29) (width 1) (layer B.Cu) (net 8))
 (segment (start 128.92 66.924402) (end 124.385576 62.38998) (width 1) (layer B.Cu) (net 8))
 (segment (start 109.982 66.29) (end 109.982 68.14) (width 1) (layer B.Cu) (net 8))
 (segment (start 124.385576 62.38998) (end 113.88202 62.38998) (width 1) (layer B.Cu) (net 8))
 (segment (start 128.92 68.14) (end 128.92 66.924402) (width 1) (layer B.Cu) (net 8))
 (segment (start 113.83 88.34) (end 114.07 88.1) (width 0.5) (layer F.Cu) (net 4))
 (segment (start 106.475 88.34) (end 113.83 88.34) (width 0.5) (layer F.Cu) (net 4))
 (segment (start 116.945 88.1) (end 119.205 90.36) (width 0.5) (layer F.Cu) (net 4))
 (segment (start 114.07 88.1) (end 116.945 88.1) (width 0.5) (layer F.Cu) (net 4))
 (segment (start 113.83 110.073332) (end 114.07 109.833332) (width 0.5) (layer F.Cu) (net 9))
 (segment (start 106.475 110.073332) (end 113.83 110.073332) (width 0.5) (layer F.Cu) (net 9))
 (segment (start 122.9 110.375) (end 123.7 110.375) (width 0.5) (layer F.Cu) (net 9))
 (segment (start 122.791667 110.483333) (end 122.9 110.375) (width 0.5) (layer F.Cu) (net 9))
 (segment (start 115.57 109.833332) (end 116.220001 110.483333) (width 0.5) (layer F.Cu) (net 9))
 (segment (start 116.220001 110.483333) (end 122.791667 110.483333) (width 0.5) (layer F.Cu) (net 9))
 (segment (start 114.07 109.833332) (end 115.57 109.833332) (width 0.5) (layer F.Cu) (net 9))
 (segment (start 113.83 99.206666) (end 114.07 98.966666) (width 0.5) (layer F.Cu) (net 14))
 (segment (start 106.475 99.206666) (end 113.83 99.206666) (width 0.5) (layer F.Cu) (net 14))
 (segment (start 116.789166 98.966666) (end 119.2025 101.38) (width 0.5) (layer F.Cu) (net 14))
 (segment (start 114.07 98.966666) (end 116.789166 98.966666) (width 0.5) (layer F.Cu) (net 14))
 (segment (start 109.6225 83.26) (end 109.8 83.0825) (width 0.5) (layer F.Cu) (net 26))
 (segment (start 106.475 83.26) (end 109.6225 83.26) (width 0.5) (layer F.Cu) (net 26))
 (segment (start 109.696668 104.993332) (end 109.85 104.84) (width 0.5) (layer F.Cu) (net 27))
 (segment (start 106.475 104.993332) (end 109.696668 104.993332) (width 0.5) (layer F.Cu) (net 27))
 (segment (start 109.695834 94.126666) (end 109.84 93.9825) (width 0.5) (layer F.Cu) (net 28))
 (segment (start 106.475 94.126666) (end 109.695834 94.126666) (width 0.5) (layer F.Cu) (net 28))
 (segment (start 111.985 71.535) (end 112 71.55) (width 0.5) (layer F.Cu) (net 30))
 (segment (start 109.84 71.535) (end 111.985 71.535) (width 0.5) (layer F.Cu) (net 30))
 (segment (start 112 72.35) (end 112 71.55) (width 0.5) (layer F.Cu) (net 30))
 (segment (start 110.832144 74.94751) (end 112 73.779654) (width 0.5) (layer F.Cu) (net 30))
 (segment (start 112 73.779654) (end 112 72.35) (width 0.5) (layer F.Cu) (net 30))
 (segment (start 110.55249 74.94751) (end 110.832144 74.94751) (width 0.5) (layer F.Cu) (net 30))
 (segment (start 109.95 75.55) (end 110.55249 74.94751) (width 0.5) (layer F.Cu) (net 30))
 (segment (start 112.57 79.22) (end 114.07 79.22) (width 0.5) (layer F.Cu) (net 19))
 (segment (start 108.215 79.22) (end 112.57 79.22) (width 0.5) (layer F.Cu) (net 19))
 (segment (start 106.585 77.59) (end 108.215 79.22) (width 0.5) (layer F.Cu) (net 19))
 (segment (start 106.475 77.59) (end 106.585 77.59) (width 0.5) (layer F.Cu) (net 19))
 (segment (start 108.875 73.41) (end 109.04 73.41) (width 0.5) (layer F.Cu) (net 29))
 (segment (start 109.04 73.41) (end 109.84 73.41) (width 0.5) (layer F.Cu) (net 29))
 (segment (start 107.975 72.51) (end 108.875 73.41) (width 0.5) (layer F.Cu) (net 29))
 (segment (start 106.475 72.51) (end 107.975 72.51) (width 0.5) (layer F.Cu) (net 29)))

